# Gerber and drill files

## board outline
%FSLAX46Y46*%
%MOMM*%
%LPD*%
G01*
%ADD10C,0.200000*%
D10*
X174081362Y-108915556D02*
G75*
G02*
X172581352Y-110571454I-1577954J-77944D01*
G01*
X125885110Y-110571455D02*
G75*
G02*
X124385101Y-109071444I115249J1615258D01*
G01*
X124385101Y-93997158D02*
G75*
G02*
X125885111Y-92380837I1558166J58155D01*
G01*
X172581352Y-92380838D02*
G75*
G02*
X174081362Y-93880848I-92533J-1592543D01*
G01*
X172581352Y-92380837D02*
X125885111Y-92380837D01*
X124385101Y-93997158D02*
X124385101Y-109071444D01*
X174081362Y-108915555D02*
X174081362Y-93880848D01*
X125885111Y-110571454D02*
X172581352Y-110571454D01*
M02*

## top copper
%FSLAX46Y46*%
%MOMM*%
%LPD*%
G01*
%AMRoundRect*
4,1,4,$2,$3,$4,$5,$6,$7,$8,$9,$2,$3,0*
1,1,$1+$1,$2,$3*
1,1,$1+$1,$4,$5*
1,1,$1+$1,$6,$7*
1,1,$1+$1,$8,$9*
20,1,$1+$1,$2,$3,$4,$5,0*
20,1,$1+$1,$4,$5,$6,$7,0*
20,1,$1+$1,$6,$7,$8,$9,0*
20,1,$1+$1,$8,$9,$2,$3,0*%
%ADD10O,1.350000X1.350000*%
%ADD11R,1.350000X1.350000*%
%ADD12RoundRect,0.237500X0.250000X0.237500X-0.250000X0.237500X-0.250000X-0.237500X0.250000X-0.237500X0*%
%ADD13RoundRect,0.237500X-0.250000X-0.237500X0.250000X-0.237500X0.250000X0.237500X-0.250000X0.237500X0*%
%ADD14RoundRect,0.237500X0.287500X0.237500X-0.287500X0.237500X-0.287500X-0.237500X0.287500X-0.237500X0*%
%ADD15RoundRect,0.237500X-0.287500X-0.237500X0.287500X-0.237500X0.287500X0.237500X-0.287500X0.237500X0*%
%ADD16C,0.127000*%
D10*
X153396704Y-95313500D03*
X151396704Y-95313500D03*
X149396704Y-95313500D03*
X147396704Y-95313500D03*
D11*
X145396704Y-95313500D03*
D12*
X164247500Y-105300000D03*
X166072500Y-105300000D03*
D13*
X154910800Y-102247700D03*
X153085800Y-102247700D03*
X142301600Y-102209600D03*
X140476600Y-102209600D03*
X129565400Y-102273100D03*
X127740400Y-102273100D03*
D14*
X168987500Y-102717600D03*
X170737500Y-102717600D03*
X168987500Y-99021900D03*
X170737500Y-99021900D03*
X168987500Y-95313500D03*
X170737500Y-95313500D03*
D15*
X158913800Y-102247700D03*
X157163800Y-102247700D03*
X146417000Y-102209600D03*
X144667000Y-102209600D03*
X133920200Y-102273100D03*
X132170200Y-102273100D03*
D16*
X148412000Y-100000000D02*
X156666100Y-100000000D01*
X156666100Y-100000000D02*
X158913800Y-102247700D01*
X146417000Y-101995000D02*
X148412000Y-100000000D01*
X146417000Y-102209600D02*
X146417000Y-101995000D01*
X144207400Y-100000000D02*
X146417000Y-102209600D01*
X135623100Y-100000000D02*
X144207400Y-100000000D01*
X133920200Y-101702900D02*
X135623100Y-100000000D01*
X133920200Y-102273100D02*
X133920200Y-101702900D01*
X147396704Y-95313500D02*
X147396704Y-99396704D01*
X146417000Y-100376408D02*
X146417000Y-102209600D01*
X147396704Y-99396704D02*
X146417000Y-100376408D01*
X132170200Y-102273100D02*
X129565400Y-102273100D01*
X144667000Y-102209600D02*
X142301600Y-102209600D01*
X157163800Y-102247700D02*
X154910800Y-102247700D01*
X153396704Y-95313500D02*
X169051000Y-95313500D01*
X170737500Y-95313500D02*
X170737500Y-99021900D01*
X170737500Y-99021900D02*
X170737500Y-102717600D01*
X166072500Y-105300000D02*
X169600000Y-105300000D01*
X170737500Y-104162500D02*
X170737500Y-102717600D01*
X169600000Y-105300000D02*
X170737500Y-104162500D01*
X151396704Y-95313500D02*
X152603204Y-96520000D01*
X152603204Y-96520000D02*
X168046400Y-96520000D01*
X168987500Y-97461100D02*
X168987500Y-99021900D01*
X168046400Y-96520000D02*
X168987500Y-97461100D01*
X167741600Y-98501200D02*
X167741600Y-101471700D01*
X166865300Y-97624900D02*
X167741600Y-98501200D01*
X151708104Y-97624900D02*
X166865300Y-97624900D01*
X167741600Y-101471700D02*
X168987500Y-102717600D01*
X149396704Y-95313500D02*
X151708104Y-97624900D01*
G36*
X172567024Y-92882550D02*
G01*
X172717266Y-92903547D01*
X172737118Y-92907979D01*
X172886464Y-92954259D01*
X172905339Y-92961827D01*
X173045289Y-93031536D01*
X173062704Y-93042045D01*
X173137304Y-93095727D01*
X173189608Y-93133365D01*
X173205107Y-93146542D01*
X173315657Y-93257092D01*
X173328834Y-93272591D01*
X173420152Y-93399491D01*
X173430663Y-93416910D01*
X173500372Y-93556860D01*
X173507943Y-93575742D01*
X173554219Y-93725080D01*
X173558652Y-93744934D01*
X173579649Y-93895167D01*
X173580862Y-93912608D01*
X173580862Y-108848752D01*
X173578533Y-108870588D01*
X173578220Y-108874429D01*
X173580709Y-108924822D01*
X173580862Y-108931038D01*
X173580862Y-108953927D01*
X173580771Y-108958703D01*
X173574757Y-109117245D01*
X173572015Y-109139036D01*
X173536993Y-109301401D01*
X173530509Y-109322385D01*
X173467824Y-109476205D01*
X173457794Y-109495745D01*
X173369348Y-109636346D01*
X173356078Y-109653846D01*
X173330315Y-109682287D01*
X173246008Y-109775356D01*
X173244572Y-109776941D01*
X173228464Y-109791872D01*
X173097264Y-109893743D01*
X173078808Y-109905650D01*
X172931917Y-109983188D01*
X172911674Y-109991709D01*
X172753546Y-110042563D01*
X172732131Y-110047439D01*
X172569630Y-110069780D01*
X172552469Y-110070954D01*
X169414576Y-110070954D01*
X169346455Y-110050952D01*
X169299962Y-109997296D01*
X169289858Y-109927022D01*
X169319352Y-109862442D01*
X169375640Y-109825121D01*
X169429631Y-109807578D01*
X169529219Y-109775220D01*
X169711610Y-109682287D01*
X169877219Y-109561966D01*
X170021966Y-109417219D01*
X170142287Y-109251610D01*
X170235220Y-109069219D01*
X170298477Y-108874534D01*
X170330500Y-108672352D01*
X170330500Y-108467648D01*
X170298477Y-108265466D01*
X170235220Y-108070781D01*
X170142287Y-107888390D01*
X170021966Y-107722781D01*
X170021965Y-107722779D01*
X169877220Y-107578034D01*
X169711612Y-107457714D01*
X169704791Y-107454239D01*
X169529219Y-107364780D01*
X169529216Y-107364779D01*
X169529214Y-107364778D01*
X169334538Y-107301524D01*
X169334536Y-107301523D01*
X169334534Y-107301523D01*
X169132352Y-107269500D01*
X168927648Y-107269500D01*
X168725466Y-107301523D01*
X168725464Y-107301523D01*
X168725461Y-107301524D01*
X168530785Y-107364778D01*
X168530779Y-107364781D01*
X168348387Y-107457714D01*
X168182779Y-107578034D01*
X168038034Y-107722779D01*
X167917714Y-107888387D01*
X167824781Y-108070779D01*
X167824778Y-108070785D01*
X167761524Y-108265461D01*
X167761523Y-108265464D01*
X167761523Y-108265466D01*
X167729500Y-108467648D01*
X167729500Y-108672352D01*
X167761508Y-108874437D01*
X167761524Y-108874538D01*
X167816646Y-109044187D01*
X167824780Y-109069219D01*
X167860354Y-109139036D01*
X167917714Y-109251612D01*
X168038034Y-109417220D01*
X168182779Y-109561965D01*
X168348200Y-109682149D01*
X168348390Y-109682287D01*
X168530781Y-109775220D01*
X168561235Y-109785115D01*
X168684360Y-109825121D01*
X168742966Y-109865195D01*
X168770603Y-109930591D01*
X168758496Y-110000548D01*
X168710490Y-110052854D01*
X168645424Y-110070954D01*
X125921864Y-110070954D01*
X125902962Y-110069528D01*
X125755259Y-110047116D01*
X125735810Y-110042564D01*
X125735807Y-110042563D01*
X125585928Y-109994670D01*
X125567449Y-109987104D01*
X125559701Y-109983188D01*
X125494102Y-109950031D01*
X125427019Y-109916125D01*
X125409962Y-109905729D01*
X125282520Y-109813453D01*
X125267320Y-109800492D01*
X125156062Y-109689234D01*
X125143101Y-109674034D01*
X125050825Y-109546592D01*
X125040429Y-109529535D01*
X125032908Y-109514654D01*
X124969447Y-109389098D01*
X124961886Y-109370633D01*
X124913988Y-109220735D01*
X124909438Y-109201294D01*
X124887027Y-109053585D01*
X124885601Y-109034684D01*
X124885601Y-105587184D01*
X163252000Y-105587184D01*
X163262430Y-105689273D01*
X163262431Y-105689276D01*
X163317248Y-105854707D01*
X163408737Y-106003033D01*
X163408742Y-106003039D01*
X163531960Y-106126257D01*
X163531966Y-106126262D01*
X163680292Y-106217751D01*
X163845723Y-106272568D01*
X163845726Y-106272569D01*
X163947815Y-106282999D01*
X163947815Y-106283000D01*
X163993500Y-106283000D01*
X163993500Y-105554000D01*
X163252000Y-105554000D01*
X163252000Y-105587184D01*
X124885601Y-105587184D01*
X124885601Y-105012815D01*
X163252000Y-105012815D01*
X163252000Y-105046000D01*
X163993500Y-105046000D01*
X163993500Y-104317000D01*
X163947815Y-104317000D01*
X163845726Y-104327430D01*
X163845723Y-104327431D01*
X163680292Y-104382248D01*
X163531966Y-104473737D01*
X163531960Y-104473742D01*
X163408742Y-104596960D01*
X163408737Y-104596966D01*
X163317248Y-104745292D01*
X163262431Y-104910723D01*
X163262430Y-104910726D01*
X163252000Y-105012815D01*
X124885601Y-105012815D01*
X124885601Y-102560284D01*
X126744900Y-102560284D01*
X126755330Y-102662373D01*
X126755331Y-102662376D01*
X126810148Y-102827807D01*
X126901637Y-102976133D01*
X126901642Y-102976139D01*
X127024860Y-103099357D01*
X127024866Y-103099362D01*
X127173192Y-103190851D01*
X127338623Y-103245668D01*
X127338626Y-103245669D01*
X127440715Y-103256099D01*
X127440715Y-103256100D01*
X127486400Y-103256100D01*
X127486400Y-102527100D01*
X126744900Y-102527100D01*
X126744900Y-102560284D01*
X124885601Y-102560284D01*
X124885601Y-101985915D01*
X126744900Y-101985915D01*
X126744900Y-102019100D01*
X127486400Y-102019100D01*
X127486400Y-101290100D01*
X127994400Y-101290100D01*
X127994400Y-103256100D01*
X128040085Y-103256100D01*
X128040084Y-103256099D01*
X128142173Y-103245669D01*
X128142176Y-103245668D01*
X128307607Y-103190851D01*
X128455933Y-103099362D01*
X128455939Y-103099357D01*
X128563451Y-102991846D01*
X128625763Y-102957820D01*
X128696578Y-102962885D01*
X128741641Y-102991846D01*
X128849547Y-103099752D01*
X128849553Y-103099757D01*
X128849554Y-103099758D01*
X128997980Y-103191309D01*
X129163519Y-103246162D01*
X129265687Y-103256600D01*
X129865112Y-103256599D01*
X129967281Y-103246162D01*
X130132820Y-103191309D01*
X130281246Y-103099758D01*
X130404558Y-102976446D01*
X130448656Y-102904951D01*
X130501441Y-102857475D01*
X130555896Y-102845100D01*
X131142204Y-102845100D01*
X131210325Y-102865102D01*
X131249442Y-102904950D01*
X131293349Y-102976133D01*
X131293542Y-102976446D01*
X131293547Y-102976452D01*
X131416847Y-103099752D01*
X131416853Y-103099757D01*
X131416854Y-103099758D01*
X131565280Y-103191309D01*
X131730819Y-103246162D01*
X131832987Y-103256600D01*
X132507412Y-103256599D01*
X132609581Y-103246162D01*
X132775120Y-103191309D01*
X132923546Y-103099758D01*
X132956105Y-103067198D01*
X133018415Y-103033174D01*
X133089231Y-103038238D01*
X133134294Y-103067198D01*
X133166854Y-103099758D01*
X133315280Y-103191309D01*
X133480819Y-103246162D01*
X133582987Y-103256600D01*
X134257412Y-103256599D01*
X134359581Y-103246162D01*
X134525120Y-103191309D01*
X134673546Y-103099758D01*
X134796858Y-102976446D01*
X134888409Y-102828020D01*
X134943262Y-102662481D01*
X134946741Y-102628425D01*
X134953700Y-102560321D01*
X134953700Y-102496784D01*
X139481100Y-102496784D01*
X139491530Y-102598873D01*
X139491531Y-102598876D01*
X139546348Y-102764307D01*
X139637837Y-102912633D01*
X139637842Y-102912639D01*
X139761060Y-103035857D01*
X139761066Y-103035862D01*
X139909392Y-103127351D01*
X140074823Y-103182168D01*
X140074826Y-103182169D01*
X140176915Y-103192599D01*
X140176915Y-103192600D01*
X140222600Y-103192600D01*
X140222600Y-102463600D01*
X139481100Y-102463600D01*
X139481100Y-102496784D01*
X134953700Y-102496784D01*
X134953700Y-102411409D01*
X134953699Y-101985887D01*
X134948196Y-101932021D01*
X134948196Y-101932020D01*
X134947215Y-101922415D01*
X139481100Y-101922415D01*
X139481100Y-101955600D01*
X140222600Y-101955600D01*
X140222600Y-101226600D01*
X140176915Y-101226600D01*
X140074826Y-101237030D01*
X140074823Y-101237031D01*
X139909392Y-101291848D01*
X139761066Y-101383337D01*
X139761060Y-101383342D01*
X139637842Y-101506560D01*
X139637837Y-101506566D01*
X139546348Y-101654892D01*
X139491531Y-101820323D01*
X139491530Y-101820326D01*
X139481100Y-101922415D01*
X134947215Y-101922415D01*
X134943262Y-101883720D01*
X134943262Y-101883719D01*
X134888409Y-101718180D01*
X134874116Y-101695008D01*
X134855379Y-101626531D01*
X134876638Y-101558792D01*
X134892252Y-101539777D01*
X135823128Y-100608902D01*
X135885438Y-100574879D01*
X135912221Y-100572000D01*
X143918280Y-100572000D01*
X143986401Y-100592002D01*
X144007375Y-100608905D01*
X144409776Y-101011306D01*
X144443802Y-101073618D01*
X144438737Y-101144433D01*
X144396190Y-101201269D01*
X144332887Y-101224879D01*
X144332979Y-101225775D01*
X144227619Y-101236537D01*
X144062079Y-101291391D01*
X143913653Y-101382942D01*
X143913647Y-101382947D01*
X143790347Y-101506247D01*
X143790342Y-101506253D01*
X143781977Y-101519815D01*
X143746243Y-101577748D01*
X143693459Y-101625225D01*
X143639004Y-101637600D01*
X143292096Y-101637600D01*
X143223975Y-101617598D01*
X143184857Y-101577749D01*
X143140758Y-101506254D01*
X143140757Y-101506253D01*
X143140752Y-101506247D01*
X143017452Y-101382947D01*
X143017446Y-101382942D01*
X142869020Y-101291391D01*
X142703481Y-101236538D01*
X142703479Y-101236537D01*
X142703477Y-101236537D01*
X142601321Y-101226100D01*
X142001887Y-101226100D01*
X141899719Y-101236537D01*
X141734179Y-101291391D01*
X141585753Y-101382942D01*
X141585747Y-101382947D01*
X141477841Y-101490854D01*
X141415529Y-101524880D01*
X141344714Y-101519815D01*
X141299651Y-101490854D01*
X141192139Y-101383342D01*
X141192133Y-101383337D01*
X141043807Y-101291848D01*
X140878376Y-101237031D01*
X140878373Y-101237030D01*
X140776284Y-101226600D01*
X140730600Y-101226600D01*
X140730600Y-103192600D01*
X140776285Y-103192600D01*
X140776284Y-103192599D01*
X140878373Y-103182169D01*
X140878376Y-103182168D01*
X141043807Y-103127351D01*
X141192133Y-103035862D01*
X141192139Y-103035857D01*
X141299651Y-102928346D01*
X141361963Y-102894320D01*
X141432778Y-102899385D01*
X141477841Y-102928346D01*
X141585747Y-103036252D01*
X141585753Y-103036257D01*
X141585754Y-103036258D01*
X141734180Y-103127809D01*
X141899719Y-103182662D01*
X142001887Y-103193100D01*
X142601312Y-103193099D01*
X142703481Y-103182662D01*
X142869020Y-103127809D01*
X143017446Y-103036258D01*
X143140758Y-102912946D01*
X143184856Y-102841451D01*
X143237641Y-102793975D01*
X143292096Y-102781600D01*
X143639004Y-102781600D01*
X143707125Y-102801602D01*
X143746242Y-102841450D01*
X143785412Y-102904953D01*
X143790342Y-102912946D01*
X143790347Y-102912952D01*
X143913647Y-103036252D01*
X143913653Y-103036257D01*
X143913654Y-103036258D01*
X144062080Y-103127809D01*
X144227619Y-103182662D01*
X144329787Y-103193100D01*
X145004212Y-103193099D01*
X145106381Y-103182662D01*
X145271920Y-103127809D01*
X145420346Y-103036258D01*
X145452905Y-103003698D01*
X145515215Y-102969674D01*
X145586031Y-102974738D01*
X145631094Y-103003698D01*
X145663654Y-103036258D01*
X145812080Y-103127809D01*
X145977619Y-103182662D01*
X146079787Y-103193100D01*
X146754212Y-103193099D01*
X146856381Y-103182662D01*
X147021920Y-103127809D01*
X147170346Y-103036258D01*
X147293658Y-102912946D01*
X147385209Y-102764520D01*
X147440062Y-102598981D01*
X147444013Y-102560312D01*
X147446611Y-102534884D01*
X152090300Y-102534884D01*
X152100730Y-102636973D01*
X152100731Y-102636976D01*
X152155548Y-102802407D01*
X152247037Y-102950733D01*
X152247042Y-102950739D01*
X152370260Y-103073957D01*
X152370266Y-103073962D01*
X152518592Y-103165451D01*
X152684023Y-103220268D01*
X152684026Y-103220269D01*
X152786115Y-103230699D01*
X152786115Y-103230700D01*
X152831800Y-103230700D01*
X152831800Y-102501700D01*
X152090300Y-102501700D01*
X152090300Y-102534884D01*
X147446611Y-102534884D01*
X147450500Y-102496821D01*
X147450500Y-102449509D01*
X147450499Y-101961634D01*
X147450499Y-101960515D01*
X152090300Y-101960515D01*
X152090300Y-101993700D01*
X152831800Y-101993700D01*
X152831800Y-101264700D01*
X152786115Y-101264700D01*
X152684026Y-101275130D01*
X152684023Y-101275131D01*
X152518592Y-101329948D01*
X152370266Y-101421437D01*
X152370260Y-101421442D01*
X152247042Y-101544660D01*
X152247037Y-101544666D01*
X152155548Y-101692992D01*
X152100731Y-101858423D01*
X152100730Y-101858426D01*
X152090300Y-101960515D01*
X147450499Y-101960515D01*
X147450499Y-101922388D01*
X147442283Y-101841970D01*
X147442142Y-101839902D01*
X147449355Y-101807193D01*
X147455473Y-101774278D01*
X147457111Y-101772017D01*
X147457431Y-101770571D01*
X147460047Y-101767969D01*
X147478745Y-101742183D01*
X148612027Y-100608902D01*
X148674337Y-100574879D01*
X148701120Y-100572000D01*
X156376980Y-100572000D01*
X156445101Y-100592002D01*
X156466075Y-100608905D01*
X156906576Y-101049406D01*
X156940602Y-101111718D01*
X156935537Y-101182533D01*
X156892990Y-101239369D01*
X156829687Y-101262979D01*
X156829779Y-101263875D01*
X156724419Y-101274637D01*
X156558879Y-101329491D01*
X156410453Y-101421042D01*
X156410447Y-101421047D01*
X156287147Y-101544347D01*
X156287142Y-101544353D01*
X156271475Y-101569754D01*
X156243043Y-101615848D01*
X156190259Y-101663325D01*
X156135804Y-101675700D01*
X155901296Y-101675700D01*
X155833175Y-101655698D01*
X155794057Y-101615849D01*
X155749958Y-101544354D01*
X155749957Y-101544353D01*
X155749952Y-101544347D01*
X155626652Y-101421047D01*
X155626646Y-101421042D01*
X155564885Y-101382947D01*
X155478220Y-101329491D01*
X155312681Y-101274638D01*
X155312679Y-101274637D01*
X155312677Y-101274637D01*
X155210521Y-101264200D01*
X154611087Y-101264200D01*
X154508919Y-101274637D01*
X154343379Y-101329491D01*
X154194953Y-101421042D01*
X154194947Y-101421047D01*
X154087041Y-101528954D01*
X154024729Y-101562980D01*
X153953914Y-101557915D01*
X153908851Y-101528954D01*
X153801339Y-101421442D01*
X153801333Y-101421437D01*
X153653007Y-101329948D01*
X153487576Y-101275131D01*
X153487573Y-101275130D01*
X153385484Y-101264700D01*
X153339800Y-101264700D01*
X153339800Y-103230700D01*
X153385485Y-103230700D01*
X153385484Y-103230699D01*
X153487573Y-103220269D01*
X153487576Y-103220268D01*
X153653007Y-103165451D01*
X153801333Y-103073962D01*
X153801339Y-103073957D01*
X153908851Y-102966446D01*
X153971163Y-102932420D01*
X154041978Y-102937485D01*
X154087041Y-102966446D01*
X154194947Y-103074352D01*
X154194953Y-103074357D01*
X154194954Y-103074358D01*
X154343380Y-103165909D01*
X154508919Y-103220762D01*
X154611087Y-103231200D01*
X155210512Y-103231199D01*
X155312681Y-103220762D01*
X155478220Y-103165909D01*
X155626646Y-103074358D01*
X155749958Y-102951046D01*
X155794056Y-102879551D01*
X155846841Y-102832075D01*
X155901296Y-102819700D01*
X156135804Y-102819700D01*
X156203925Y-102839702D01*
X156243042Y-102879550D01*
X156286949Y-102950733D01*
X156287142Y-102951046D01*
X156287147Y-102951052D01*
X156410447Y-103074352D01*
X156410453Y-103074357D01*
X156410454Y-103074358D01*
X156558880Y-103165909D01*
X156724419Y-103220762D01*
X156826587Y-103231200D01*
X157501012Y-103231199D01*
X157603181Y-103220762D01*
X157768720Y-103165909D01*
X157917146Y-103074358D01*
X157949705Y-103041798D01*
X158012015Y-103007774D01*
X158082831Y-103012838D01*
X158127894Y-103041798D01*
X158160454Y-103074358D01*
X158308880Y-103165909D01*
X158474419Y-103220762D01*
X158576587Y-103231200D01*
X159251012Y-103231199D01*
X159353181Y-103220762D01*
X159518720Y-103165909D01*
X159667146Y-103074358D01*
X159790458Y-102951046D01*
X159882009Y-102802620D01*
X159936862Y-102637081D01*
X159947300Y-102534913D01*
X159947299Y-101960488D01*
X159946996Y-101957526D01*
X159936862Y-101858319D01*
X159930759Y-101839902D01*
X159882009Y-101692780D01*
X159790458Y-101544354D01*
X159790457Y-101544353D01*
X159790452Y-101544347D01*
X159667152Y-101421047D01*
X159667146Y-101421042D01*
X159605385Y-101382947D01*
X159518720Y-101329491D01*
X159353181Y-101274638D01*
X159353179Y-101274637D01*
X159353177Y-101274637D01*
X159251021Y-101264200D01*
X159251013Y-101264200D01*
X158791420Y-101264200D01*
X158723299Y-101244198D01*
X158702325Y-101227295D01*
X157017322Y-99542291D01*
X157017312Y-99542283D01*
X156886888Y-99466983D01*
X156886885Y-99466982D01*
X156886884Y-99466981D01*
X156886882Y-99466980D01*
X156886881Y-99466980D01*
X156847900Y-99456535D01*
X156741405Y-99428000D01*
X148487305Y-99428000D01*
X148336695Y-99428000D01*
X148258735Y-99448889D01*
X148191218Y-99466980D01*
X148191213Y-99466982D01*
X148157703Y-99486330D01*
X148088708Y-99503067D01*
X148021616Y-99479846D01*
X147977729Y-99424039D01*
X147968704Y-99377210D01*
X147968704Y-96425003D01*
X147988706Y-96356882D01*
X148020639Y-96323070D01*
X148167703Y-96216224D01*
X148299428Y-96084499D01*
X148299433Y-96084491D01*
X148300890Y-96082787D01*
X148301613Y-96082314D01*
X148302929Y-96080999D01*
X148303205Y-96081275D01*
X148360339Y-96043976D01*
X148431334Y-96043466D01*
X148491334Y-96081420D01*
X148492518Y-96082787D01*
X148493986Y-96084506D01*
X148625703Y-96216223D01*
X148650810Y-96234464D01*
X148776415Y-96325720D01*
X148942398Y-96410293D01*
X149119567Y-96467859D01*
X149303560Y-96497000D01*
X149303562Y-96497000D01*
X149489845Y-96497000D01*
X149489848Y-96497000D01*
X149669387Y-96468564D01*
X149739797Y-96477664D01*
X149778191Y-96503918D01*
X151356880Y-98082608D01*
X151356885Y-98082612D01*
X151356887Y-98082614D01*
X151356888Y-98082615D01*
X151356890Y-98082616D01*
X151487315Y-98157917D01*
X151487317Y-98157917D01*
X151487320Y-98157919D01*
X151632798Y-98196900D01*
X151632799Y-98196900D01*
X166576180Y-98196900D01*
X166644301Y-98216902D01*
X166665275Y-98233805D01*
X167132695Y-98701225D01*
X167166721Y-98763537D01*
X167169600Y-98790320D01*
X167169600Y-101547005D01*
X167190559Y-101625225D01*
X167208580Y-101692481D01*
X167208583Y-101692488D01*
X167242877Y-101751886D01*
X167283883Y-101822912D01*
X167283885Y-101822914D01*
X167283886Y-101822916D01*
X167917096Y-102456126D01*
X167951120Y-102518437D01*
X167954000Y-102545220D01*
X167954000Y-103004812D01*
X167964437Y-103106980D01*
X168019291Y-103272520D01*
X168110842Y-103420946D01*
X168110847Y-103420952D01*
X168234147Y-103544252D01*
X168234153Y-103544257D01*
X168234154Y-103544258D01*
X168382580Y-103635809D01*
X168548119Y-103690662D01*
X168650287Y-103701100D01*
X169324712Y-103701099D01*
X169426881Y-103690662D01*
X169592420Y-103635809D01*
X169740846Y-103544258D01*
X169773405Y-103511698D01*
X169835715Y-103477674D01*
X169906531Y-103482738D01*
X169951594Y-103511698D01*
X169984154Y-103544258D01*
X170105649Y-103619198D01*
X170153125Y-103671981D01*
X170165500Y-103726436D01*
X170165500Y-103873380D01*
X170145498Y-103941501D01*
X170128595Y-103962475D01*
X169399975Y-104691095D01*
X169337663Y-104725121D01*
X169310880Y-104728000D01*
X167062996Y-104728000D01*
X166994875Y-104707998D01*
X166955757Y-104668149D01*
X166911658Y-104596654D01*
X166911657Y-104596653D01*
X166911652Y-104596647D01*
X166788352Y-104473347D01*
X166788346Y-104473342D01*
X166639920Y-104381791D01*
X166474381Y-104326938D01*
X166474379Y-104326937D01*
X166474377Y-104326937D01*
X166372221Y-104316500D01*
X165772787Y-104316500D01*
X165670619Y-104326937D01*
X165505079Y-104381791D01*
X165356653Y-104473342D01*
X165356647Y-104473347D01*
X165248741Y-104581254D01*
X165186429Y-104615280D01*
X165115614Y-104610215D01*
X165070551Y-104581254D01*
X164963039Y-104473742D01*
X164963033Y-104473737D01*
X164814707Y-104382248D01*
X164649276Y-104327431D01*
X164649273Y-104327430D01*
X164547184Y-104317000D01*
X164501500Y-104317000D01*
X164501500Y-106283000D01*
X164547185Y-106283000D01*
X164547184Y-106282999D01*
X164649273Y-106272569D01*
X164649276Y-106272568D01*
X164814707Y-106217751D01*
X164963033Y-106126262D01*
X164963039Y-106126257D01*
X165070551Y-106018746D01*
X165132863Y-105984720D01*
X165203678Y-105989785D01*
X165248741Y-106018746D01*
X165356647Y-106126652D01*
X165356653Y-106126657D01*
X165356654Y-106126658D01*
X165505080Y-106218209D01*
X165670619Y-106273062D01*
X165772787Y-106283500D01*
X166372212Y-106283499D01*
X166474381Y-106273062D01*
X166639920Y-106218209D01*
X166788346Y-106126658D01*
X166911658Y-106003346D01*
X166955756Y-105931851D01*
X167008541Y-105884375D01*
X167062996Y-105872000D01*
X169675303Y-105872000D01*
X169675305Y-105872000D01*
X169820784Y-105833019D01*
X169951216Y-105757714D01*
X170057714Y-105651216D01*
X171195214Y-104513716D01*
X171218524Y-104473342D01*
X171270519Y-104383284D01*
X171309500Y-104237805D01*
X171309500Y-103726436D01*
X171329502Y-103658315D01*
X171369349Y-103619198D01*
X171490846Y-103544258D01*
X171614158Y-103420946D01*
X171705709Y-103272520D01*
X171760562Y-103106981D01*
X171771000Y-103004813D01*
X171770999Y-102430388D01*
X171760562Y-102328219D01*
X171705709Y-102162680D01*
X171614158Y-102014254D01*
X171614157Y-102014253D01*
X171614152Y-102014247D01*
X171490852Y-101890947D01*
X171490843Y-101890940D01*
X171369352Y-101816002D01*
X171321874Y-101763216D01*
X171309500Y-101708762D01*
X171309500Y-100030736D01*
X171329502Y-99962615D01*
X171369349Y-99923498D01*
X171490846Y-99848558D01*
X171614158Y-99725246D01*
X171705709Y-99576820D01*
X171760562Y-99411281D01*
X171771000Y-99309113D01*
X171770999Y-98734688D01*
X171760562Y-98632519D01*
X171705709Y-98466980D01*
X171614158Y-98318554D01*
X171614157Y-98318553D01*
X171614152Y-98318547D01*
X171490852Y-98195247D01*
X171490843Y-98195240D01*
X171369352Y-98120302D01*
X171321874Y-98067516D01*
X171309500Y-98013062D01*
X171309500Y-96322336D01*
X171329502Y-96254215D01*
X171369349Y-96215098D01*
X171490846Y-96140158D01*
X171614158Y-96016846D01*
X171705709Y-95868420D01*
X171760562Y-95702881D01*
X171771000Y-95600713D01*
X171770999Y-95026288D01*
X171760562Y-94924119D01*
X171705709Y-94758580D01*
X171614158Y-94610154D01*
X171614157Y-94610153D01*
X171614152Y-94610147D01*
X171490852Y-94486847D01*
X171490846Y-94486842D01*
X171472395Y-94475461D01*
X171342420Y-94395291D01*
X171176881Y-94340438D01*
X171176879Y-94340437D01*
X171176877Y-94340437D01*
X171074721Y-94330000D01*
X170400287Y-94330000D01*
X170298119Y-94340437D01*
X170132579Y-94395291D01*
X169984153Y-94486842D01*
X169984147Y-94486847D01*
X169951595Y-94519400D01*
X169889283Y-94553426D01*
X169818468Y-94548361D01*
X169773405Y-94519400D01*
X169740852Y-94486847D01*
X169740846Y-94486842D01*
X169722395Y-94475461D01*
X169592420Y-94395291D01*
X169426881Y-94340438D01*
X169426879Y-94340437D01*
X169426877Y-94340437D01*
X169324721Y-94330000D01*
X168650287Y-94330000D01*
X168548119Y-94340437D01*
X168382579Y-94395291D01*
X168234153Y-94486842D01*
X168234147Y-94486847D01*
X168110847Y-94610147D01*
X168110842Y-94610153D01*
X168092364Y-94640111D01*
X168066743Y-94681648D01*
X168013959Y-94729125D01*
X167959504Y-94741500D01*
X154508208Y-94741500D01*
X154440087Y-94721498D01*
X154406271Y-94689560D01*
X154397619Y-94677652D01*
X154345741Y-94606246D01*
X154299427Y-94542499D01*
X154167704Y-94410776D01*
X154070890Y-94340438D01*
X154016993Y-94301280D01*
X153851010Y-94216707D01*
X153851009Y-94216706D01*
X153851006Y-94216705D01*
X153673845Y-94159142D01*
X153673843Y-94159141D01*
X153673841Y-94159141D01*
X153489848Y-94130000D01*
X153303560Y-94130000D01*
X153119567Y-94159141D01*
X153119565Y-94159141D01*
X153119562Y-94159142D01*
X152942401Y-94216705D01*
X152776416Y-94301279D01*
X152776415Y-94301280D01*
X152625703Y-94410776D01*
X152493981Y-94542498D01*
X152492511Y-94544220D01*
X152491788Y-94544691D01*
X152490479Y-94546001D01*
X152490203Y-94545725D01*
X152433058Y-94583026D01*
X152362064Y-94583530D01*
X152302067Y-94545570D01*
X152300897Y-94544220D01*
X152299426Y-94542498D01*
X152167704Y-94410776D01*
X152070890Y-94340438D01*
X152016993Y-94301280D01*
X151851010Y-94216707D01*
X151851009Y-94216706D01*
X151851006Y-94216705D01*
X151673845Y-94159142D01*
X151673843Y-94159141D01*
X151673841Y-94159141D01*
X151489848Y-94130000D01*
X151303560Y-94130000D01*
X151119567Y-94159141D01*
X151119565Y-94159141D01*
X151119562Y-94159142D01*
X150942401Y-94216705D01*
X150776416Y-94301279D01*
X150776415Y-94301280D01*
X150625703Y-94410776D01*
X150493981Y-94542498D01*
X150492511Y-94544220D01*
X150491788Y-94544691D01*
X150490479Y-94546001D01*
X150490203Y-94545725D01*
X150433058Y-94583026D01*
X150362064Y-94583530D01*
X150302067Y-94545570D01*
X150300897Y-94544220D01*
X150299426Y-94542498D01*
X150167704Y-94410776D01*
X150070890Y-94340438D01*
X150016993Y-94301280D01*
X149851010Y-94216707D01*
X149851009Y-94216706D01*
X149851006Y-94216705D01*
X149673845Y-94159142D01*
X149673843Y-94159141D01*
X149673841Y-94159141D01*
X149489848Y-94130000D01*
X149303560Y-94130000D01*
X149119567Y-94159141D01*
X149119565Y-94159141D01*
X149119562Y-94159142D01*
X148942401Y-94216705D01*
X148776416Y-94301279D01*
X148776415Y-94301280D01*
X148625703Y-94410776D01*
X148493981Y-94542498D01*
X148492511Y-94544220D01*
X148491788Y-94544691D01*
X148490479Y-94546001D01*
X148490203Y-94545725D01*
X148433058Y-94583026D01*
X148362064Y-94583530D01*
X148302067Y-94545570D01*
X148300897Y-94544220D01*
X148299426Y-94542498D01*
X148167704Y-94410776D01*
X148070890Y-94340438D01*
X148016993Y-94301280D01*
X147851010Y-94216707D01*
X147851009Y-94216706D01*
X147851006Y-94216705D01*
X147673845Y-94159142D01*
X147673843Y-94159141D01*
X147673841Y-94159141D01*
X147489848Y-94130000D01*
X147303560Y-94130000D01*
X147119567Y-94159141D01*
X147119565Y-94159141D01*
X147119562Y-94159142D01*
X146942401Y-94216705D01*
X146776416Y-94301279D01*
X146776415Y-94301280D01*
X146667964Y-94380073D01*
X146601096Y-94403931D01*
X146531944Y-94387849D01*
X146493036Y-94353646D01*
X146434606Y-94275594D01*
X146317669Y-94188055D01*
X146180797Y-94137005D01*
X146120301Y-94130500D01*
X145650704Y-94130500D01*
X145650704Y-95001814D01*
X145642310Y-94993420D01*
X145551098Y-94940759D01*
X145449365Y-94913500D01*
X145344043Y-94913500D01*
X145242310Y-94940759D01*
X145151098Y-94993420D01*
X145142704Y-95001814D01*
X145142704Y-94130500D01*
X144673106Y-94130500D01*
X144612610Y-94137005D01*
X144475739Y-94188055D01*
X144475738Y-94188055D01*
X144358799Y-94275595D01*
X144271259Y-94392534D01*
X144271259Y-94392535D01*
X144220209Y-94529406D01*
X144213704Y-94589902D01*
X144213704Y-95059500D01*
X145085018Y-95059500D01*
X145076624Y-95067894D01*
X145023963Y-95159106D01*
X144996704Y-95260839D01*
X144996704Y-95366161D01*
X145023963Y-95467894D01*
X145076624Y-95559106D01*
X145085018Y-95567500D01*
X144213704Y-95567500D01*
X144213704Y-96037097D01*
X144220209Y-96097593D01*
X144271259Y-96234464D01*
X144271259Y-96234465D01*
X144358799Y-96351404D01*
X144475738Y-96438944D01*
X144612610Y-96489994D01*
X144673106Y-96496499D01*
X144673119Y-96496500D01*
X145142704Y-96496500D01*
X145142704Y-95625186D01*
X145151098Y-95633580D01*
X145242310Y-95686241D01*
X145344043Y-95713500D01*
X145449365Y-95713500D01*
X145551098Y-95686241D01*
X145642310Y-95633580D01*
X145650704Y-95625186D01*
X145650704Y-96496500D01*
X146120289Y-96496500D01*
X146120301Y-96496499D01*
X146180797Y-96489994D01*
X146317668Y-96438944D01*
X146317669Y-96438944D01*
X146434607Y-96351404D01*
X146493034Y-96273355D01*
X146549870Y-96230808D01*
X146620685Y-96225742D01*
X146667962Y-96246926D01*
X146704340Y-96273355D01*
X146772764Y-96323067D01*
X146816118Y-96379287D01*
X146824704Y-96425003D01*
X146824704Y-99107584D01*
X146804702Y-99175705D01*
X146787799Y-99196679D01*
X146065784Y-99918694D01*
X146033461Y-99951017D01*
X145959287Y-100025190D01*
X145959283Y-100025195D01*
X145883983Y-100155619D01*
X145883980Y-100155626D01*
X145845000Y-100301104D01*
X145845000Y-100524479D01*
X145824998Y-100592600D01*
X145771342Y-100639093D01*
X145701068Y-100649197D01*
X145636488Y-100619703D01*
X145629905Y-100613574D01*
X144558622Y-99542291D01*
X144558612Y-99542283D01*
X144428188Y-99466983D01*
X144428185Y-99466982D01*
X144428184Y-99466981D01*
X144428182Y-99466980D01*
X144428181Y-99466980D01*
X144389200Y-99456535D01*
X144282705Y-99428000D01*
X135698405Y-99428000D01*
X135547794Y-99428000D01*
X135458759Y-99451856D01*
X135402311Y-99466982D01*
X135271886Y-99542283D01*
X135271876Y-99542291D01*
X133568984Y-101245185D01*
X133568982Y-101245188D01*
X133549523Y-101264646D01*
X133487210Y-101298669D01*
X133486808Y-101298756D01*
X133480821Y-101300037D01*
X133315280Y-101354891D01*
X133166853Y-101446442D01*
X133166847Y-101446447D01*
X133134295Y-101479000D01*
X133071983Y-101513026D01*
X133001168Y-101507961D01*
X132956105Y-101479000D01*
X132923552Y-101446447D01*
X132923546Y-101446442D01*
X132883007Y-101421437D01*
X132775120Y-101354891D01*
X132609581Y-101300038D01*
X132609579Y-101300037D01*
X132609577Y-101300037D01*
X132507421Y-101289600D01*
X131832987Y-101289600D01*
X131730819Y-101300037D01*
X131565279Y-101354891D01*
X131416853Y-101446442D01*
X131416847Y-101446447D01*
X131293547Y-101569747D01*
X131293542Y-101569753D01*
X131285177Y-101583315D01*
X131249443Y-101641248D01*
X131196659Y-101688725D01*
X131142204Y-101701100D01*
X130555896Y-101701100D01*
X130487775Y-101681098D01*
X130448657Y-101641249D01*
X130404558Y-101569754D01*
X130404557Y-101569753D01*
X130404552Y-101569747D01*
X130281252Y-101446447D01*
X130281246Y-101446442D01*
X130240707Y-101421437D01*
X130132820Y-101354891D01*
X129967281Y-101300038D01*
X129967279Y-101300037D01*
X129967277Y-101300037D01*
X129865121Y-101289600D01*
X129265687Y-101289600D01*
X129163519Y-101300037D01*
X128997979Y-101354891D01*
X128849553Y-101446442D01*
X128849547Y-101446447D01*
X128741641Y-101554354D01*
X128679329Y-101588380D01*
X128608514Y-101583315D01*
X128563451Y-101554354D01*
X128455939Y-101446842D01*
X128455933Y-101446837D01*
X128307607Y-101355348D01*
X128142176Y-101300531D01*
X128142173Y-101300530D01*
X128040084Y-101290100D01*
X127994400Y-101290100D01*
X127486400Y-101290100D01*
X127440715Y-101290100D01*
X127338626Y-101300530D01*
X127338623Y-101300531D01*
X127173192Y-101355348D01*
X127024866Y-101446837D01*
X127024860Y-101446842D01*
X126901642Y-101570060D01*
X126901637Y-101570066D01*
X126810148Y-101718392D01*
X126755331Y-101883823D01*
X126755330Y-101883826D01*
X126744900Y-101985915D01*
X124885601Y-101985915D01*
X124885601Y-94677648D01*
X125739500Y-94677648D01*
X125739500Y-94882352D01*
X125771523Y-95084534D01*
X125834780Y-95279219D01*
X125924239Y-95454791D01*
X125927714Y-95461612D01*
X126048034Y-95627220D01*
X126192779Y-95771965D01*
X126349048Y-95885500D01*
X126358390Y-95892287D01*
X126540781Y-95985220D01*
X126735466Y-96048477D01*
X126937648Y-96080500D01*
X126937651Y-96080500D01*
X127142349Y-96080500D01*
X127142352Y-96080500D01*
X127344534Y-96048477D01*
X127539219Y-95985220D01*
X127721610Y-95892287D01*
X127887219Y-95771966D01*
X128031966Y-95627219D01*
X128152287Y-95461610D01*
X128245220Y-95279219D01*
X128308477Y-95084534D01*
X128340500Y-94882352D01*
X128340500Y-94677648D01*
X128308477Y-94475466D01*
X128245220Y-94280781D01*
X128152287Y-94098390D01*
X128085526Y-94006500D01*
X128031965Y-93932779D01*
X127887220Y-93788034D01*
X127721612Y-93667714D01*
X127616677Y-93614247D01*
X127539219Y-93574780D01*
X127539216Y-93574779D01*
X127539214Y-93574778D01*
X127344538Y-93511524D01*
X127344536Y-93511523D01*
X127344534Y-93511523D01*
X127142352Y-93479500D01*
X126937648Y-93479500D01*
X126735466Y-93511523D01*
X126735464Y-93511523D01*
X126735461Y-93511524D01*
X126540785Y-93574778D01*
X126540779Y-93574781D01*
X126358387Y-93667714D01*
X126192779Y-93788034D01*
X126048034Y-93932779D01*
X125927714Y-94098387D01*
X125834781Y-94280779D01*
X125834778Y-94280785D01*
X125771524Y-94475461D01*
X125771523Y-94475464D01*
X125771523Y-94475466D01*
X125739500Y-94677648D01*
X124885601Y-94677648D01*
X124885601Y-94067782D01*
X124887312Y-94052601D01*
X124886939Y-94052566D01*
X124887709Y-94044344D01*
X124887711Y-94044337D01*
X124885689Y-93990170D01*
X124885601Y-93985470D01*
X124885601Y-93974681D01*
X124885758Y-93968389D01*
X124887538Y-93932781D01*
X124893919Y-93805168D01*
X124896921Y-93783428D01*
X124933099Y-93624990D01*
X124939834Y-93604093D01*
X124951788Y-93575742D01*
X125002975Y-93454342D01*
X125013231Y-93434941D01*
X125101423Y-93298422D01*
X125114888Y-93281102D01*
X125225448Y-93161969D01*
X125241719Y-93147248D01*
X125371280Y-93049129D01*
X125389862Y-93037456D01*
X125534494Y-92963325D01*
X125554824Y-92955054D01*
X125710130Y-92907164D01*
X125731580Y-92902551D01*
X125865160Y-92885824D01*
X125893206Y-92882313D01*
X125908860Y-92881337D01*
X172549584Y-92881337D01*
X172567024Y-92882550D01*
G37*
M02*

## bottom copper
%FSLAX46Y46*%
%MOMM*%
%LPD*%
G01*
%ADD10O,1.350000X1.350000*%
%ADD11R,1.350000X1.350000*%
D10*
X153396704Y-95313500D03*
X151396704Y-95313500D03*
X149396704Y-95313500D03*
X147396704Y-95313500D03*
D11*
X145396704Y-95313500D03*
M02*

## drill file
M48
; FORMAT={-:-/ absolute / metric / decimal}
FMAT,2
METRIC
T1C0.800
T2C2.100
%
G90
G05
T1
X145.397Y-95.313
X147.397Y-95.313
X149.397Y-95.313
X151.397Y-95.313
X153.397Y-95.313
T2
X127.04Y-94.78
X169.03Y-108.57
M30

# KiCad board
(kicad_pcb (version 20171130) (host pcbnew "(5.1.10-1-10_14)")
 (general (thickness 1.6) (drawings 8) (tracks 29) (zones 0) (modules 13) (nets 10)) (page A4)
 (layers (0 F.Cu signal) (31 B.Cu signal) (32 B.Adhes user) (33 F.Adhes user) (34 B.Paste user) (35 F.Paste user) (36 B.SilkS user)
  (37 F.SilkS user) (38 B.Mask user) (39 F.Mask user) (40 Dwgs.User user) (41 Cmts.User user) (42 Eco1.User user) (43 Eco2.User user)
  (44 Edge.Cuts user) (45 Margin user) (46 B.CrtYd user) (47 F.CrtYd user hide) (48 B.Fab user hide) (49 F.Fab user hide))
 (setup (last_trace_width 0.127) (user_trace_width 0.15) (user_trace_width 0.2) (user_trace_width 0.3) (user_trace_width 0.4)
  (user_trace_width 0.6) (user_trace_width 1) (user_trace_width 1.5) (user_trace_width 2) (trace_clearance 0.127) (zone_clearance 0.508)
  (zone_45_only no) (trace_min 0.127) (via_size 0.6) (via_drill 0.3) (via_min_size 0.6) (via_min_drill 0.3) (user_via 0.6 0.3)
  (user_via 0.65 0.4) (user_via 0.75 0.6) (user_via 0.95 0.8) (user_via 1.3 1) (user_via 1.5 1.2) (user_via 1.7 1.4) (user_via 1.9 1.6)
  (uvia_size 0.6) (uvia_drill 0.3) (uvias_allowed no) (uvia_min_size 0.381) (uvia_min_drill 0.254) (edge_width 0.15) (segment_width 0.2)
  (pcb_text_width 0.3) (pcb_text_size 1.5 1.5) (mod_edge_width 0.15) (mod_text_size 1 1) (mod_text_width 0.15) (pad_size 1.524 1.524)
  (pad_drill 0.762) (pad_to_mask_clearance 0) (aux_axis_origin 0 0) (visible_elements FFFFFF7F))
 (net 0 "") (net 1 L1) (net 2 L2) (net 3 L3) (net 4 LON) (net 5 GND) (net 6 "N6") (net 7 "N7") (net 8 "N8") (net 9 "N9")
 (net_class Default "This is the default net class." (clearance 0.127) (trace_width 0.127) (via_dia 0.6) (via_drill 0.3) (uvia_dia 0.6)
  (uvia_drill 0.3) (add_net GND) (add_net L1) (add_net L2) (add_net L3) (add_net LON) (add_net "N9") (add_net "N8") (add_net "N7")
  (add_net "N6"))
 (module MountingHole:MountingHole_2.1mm (layer F.Cu) (at 169.03 108.57)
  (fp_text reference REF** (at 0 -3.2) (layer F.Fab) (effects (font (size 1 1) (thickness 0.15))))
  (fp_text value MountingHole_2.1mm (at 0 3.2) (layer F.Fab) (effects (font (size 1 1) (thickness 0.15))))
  (pad "" np_thru_hole circle (at 0 0) (size 2.1 2.1) (drill 2.1) (layers *.Cu *.Mask)))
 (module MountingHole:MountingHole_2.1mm (layer F.Cu) (at 127.04 94.78)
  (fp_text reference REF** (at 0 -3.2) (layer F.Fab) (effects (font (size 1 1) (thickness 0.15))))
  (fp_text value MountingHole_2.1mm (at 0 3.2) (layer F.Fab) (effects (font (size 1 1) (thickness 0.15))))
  (pad "" np_thru_hole circle (at 0 0) (size 2.1 2.1) (drill 2.1) (layers *.Cu *.Mask)))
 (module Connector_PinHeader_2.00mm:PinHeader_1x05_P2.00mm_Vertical (layer F.Cu) (at 145.396704 95.3135 90)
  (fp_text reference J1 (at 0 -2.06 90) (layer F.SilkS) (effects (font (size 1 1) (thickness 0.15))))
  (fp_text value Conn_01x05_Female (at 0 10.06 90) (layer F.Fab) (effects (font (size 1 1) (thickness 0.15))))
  (pad 5 thru_hole oval (at 0 8 90) (size 1.35 1.35) (drill 0.8) (layers *.Cu *.Mask) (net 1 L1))
  (pad 4 thru_hole oval (at 0 6 90) (size 1.35 1.35) (drill 0.8) (layers *.Cu *.Mask) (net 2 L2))
  (pad 3 thru_hole oval (at 0 4 90) (size 1.35 1.35) (drill 0.8) (layers *.Cu *.Mask) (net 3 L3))
  (pad 2 thru_hole oval (at 0 2 90) (size 1.35 1.35) (drill 0.8) (layers *.Cu *.Mask) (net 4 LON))
  (pad 1 thru_hole rect (at 0 0 90) (size 1.35 1.35) (drill 0.8) (layers *.Cu *.Mask) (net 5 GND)))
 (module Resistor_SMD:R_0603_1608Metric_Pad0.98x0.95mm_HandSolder (layer F.Cu) (at 165.16 105.3 180)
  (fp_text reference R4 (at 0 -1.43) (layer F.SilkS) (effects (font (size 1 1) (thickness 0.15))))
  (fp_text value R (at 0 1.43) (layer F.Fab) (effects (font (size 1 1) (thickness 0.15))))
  (pad 2 smd roundrect (at 0.9125 0 180) (size 0.975 0.95) (layers F.Cu F.Paste F.Mask) (roundrect_rratio 0.25) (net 5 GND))
  (pad 1 smd roundrect (at -0.9125 0 180) (size 0.975 0.95) (layers F.Cu F.Paste F.Mask) (roundrect_rratio 0.25) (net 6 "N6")))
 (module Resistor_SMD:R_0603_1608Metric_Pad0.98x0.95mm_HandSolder (layer F.Cu) (at 153.9983 102.2477)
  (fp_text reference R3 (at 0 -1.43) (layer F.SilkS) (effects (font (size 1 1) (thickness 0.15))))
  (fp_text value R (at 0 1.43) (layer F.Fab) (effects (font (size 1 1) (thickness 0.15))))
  (pad 2 smd roundrect (at 0.9125 0) (size 0.975 0.95) (layers F.Cu F.Paste F.Mask) (roundrect_rratio 0.25) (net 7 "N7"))
  (pad 1 smd roundrect (at -0.9125 0) (size 0.975 0.95) (layers F.Cu F.Paste F.Mask) (roundrect_rratio 0.25) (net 5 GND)))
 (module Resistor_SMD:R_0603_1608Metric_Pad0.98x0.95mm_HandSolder (layer F.Cu) (at 141.3891 102.2096)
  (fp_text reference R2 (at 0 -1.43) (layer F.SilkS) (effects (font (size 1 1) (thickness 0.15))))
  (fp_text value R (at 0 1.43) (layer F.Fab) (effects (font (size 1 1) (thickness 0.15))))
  (pad 2 smd roundrect (at 0.9125 0) (size 0.975 0.95) (layers F.Cu F.Paste F.Mask) (roundrect_rratio 0.25) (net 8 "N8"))
  (pad 1 smd roundrect (at -0.9125 0) (size 0.975 0.95) (layers F.Cu F.Paste F.Mask) (roundrect_rratio 0.25) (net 5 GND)))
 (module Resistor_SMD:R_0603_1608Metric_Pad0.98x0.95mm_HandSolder (layer F.Cu) (at 128.6529 102.2731)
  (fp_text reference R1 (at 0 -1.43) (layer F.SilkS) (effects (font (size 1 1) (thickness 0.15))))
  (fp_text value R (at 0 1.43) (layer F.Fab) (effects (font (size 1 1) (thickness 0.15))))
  (pad 2 smd roundrect (at 0.9125 0) (size 0.975 0.95) (layers F.Cu F.Paste F.Mask) (roundrect_rratio 0.25) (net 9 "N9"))
  (pad 1 smd roundrect (at -0.9125 0) (size 0.975 0.95) (layers F.Cu F.Paste F.Mask) (roundrect_rratio 0.25) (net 5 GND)))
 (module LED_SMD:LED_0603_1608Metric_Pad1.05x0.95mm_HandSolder (layer F.Cu) (at 169.8625 102.7176 180)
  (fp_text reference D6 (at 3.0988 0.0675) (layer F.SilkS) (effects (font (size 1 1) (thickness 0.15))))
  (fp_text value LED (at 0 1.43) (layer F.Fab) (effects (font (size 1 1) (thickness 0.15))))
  (pad 2 smd roundrect (at 0.875 0 180) (size 1.05 0.95) (layers F.Cu F.Paste F.Mask) (roundrect_rratio 0.25) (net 3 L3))
  (pad 1 smd roundrect (at -0.875 0 180) (size 1.05 0.95) (layers F.Cu F.Paste F.Mask) (roundrect_rratio 0.25) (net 6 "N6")))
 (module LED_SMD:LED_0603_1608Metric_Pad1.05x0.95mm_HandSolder (layer F.Cu) (at 169.8625 99.0219 180)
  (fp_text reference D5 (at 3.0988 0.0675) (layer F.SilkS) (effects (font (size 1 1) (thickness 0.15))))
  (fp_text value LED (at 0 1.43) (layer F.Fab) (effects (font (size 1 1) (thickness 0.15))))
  (pad 2 smd roundrect (at 0.875 0 180) (size 1.05 0.95) (layers F.Cu F.Paste F.Mask) (roundrect_rratio 0.25) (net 2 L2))
  (pad 1 smd roundrect (at -0.875 0 180) (size 1.05 0.95) (layers F.Cu F.Paste F.Mask) (roundrect_rratio 0.25) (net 6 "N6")))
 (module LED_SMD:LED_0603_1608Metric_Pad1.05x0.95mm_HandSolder (layer F.Cu) (at 169.8625 95.3135 180)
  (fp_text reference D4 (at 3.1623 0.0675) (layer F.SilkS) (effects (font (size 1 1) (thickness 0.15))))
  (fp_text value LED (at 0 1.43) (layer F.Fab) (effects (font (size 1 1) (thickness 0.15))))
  (pad 2 smd roundrect (at 0.875 0 180) (size 1.05 0.95) (layers F.Cu F.Paste F.Mask) (roundrect_rratio 0.25) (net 1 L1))
  (pad 1 smd roundrect (at -0.875 0 180) (size 1.05 0.95) (layers F.Cu F.Paste F.Mask) (roundrect_rratio 0.25) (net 6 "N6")))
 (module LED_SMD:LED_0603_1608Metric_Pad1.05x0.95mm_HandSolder (layer F.Cu) (at 158.0388 102.2477)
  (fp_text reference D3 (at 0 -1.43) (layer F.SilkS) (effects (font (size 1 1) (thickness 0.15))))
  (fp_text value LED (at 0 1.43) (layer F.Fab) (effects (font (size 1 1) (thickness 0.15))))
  (pad 2 smd roundrect (at 0.875 0) (size 1.05 0.95) (layers F.Cu F.Paste F.Mask) (roundrect_rratio 0.25) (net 4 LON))
  (pad 1 smd roundrect (at -0.875 0) (size 1.05 0.95) (layers F.Cu F.Paste F.Mask) (roundrect_rratio 0.25) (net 7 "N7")))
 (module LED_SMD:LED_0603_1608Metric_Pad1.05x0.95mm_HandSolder (layer F.Cu) (at 145.542 102.2096)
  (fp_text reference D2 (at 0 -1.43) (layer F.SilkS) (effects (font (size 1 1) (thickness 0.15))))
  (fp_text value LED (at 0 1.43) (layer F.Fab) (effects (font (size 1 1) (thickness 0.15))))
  (pad 2 smd roundrect (at 0.875 0) (size 1.05 0.95) (layers F.Cu F.Paste F.Mask) (roundrect_rratio 0.25) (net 4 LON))
  (pad 1 smd roundrect (at -0.875 0) (size 1.05 0.95) (layers F.Cu F.Paste F.Mask) (roundrect_rratio 0.25) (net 8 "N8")))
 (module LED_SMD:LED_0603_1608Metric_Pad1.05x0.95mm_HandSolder (layer F.Cu) (at 133.0452 102.2731)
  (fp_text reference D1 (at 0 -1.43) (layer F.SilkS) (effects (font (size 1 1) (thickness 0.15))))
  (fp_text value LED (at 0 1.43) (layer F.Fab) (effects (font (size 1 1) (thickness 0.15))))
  (pad 2 smd roundrect (at 0.875 0) (size 1.05 0.95) (layers F.Cu F.Paste F.Mask) (roundrect_rratio 0.25) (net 4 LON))
  (pad 1 smd roundrect (at -0.875 0) (size 1.05 0.95) (layers F.Cu F.Paste F.Mask) (roundrect_rratio 0.25) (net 9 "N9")))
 (gr_arc (start 172.503408 108.9935) (end 172.581352 110.571454) (angle -90) (layer Edge.Cuts) (width 0.2))
 (gr_arc (start 126.000359 108.956197) (end 124.385101 109.071444) (angle -81.8377804) (layer Edge.Cuts) (width 0.2))
 (gr_arc (start 125.943267 93.939003) (end 125.885111 92.380837) (angle -89.9999618) (layer Edge.Cuts) (width 0.2))
 (gr_arc (start 172.488819 93.973381) (end 174.081362 93.880848) (angle -83.34927126) (layer Edge.Cuts) (width 0.2))
 (gr_line (start 172.581352 92.380837) (end 125.885111 92.380837) (layer Edge.Cuts) (width 0.2))
 (gr_line (start 124.385101 93.997158) (end 124.385101 109.071444) (layer Edge.Cuts) (width 0.2))
 (gr_line (start 174.081362 108.915555) (end 174.081362 93.880848) (layer Edge.Cuts) (width 0.2))
 (gr_line (start 125.885111 110.571454) (end 172.581352 110.571454) (layer Edge.Cuts) (width 0.2))
 (segment (start 148.412 100) (end 156.6661 100) (width 0.127) (layer F.Cu) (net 4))
 (segment (start 156.6661 100) (end 158.9138 102.2477) (width 0.127) (layer F.Cu) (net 4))
 (segment (start 146.417 101.995) (end 148.412 100) (width 0.127) (layer F.Cu) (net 4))
 (segment (start 146.417 102.2096) (end 146.417 101.995) (width 0.127) (layer F.Cu) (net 4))
 (segment (start 144.2074 100) (end 146.417 102.2096) (width 0.127) (layer F.Cu) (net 4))
 (segment (start 135.6231 100) (end 144.2074 100) (width 0.127) (layer F.Cu) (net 4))
 (segment (start 133.9202 101.7029) (end 135.6231 100) (width 0.127) (layer F.Cu) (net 4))
 (segment (start 133.9202 102.2731) (end 133.9202 101.7029) (width 0.127) (layer F.Cu) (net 4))
 (segment (start 147.396704 95.3135) (end 147.396704 99.396704) (width 0.127) (layer F.Cu) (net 4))
 (segment (start 146.417 100.376408) (end 146.417 102.2096) (width 0.127) (layer F.Cu) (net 4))
 (segment (start 147.396704 99.396704) (end 146.417 100.376408) (width 0.127) (layer F.Cu) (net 4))
 (segment (start 132.1702 102.2731) (end 129.5654 102.2731) (width 0.127) (layer F.Cu) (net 9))
 (segment (start 144.667 102.2096) (end 142.3016 102.2096) (width 0.127) (layer F.Cu) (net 8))
 (segment (start 157.1638 102.2477) (end 154.9108 102.2477) (width 0.127) (layer F.Cu) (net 7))
 (segment (start 153.396704 95.3135) (end 169.051 95.3135) (width 0.127) (layer F.Cu) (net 1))
 (segment (start 170.7375 95.3135) (end 170.7375 99.0219) (width 0.127) (layer F.Cu) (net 6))
 (segment (start 170.7375 99.0219) (end 170.7375 102.7176) (width 0.127) (layer F.Cu) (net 6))
 (segment (start 166.0725 105.3) (end 169.6 105.3) (width 0.127) (layer F.Cu) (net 6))
 (segment (start 170.7375 104.1625) (end 170.7375 102.7176) (width 0.127) (layer F.Cu) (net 6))
 (segment (start 169.6 105.3) (end 170.7375 104.1625) (width 0.127) (layer F.Cu) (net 6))
 (segment (start 151.396704 95.3135) (end 152.603204 96.52) (width 0.127) (layer F.Cu) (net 2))
 (segment (start 152.603204 96.52) (end 168.0464 96.52) (width 0.127) (layer F.Cu) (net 2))
 (segment (start 168.9875 97.4611) (end 168.9875 99.0219) (width 0.127) (layer F.Cu) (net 2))
 (segment (start 168.0464 96.52) (end 168.9875 97.4611) (width 0.127) (layer F.Cu) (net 2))
 (segment (start 167.7416 98.5012) (end 167.7416 101.4717) (width 0.127) (layer F.Cu) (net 3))
 (segment (start 166.8653 97.6249) (end 167.7416 98.5012) (width 0.127) (layer F.Cu) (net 3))
 (segment (start 151.708104 97.6249) (end 166.8653 97.6249) (width 0.127) (layer F.Cu) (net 3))
 (segment (start 167.7416 101.4717) (end 168.9875 102.7176) (width 0.127) (layer F.Cu) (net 3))
 (segment (start 149.396704 95.3135) (end 151.708104 97.6249) (width 0.127) (layer F.Cu) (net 3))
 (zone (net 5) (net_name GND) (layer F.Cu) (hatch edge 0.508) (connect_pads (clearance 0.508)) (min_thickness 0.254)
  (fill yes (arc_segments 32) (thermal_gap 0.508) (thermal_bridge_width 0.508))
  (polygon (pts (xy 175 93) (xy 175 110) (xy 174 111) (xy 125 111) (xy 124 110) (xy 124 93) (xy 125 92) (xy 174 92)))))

